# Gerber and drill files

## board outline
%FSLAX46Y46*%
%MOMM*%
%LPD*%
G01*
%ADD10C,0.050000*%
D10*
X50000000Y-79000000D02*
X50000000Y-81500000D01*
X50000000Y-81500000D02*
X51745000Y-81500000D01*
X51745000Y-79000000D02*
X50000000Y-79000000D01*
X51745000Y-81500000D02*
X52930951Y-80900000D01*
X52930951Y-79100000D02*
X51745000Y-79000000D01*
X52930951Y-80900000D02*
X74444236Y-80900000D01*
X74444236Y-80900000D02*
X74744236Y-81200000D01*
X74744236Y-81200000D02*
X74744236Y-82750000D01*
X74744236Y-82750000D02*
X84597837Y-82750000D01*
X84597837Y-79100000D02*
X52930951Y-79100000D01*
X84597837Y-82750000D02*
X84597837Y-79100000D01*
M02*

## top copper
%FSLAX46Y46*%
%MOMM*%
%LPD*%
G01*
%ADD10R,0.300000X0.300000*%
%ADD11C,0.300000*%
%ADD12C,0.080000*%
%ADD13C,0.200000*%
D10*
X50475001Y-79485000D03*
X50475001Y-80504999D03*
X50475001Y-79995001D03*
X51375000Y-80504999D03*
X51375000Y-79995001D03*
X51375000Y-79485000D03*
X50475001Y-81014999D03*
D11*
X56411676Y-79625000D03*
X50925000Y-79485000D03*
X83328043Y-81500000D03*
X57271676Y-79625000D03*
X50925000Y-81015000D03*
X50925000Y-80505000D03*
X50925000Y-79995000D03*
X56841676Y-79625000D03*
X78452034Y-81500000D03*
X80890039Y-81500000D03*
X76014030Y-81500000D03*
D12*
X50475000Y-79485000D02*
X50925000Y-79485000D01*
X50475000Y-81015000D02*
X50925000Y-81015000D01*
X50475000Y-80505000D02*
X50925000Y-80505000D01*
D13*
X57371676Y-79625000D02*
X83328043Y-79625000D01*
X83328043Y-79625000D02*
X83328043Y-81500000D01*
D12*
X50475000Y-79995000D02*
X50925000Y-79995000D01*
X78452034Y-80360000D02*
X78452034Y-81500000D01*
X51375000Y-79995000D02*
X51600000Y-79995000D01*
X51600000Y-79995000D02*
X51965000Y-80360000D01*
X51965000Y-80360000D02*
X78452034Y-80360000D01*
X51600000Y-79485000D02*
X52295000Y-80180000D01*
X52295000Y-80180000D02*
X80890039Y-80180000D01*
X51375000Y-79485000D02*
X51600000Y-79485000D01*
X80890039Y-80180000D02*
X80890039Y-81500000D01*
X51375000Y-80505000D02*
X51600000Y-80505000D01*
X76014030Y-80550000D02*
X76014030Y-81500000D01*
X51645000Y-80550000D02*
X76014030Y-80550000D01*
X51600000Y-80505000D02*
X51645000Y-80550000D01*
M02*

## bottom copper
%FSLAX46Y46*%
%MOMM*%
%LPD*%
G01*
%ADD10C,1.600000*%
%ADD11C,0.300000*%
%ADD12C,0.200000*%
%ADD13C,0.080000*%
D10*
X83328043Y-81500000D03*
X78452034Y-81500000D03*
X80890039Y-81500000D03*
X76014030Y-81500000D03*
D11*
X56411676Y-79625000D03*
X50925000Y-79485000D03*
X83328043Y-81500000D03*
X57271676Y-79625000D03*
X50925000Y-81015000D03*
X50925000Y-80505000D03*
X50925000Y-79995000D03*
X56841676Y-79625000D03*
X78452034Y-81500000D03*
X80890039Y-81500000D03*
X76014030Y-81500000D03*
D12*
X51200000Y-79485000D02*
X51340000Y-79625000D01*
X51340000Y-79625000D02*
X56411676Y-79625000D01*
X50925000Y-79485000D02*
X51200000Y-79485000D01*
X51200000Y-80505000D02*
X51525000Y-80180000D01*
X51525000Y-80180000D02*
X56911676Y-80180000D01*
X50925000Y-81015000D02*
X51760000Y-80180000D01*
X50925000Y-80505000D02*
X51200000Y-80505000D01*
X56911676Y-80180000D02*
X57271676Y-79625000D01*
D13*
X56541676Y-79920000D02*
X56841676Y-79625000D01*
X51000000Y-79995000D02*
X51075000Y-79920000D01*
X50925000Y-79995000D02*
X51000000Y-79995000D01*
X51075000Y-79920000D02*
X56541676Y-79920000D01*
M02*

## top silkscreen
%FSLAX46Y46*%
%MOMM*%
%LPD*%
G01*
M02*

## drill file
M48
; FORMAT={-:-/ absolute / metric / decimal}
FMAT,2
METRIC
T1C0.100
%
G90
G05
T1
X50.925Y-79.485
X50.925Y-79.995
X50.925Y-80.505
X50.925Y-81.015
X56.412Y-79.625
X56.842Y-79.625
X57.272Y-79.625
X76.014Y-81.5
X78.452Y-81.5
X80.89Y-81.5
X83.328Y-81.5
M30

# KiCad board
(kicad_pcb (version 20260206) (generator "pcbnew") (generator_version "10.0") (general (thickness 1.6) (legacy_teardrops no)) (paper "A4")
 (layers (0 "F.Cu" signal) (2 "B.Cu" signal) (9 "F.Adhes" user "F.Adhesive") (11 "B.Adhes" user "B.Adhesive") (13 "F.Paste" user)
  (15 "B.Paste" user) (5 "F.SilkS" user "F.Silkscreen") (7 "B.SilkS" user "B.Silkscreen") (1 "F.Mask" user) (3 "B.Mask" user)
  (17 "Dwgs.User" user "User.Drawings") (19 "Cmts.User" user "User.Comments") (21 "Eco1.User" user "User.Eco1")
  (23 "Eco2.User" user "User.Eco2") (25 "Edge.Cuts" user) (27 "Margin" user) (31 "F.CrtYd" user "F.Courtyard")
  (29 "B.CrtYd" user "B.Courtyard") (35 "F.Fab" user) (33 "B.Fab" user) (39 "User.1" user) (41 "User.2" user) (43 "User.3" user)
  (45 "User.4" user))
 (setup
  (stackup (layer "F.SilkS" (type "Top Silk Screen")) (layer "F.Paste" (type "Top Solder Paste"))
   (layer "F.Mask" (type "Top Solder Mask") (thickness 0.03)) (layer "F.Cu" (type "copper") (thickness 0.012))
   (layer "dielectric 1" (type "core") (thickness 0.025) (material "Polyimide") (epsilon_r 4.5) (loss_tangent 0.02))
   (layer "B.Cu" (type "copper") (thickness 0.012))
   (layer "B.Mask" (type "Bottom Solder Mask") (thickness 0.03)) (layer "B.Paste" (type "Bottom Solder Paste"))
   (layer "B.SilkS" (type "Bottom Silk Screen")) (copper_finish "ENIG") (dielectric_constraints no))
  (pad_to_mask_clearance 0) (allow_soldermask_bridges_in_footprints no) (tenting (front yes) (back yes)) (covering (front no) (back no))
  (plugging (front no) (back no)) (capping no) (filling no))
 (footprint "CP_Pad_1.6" (layer "F.Cu") (at 83.328043 81.5)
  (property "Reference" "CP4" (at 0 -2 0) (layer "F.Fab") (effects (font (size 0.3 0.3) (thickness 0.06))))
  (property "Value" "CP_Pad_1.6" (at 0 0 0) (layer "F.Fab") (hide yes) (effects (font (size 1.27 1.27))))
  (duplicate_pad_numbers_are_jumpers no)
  (pad "1" smd circle (at 0 0) (size 1.6 1.6) (layers "B.Cu" "B.Mask") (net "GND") (solder_mask_margin 0.1)))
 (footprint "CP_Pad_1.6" (layer "F.Cu") (at 78.452034 81.5)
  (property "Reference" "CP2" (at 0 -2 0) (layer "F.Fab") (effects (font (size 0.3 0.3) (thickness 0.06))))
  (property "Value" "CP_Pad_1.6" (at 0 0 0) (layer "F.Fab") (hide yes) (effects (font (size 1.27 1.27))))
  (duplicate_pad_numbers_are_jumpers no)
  (pad "1" smd circle (at 0 0) (size 1.6 1.6) (layers "B.Cu" "B.Mask") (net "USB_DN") (solder_mask_margin 0.1)))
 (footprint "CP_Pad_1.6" (layer "F.Cu") (at 80.890039 81.5)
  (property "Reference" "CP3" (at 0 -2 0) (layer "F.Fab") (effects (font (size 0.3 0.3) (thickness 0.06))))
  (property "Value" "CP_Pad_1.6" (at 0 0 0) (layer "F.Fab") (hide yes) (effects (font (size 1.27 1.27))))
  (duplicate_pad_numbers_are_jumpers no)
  (pad "1" smd circle (at 0 0) (size 1.6 1.6) (layers "B.Cu" "B.Mask") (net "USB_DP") (solder_mask_margin 0.1)))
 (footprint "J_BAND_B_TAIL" (layer "F.Cu") (at 50.9 80.25)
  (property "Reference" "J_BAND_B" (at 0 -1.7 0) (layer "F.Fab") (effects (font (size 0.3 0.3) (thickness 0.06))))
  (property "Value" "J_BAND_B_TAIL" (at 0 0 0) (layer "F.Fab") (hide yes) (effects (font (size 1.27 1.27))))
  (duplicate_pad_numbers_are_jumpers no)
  (pad "1" smd rect (at -0.424999 -0.765) (size 0.3 0.3) (layers "F.Cu" "F.Mask") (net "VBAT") (solder_mask_margin 0.05)
   (thermal_bridge_angle 45))
  (pad "2" smd rect (at -0.424999 0.254999) (size 0.3 0.3) (layers "F.Cu" "F.Mask") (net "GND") (solder_mask_margin 0.05)
   (thermal_bridge_angle 45))
  (pad "3" smd rect (at -0.424999 -0.254999) (size 0.3 0.3) (layers "F.Cu" "F.Mask") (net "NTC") (solder_mask_margin 0.05)
   (thermal_bridge_angle 45))
  (pad "4" smd rect (at 0.475 0.254999) (size 0.3 0.3) (layers "F.Cu" "F.Mask") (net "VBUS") (solder_mask_margin 0.05)
   (thermal_bridge_angle 45))
  (pad "5" smd rect (at 0.475 -0.254999) (size 0.3 0.3) (layers "F.Cu" "F.Mask") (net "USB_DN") (solder_mask_margin 0.05)
   (thermal_bridge_angle 45))
  (pad "6" smd rect (at 0.475 -0.765) (size 0.3 0.3) (layers "F.Cu" "F.Mask") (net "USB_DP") (solder_mask_margin 0.05)
   (thermal_bridge_angle 45))
  (pad "7" smd rect (at -0.424999 0.764999) (size 0.3 0.3) (layers "F.Cu" "F.Mask") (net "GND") (solder_mask_margin 0.05)
   (thermal_bridge_angle 45)))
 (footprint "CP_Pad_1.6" (layer "F.Cu") (at 76.01403 81.5)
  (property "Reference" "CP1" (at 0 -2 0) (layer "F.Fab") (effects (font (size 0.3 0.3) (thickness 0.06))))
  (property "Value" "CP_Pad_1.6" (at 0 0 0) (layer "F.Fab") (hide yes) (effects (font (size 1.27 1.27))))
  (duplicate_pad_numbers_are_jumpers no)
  (pad "1" smd circle (at 0 0) (size 1.6 1.6) (layers "B.Cu" "B.Mask") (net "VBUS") (solder_mask_margin 0.1)))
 (gr_line (start 50 79) (end 50 81.5) (stroke (width 0.05) (type default)) (layer "Edge.Cuts"))
 (gr_line (start 50 81.5) (end 51.745 81.5) (stroke (width 0.05) (type default)) (layer "Edge.Cuts"))
 (gr_line (start 51.745 79) (end 50 79) (stroke (width 0.05) (type default)) (layer "Edge.Cuts"))
 (gr_line (start 51.745 81.5) (end 52.930951 80.9) (stroke (width 0.05) (type default)) (layer "Edge.Cuts"))
 (gr_line (start 52.930951 79.1) (end 51.745 79) (stroke (width 0.05) (type default)) (layer "Edge.Cuts"))
 (gr_line (start 52.930951 80.9) (end 74.444236 80.9) (stroke (width 0.05) (type default)) (layer "Edge.Cuts"))
 (gr_line (start 74.444236 80.9) (end 74.744236 81.2) (stroke (width 0.05) (type default)) (layer "Edge.Cuts"))
 (gr_line (start 74.744236 81.2) (end 74.744236 82.75) (stroke (width 0.05) (type default)) (layer "Edge.Cuts"))
 (gr_line (start 74.744236 82.75) (end 84.597837 82.75) (stroke (width 0.05) (type default)) (layer "Edge.Cuts"))
 (gr_line (start 84.597837 79.1) (end 52.930951 79.1) (stroke (width 0.05) (type default)) (layer "Edge.Cuts"))
 (gr_line (start 84.597837 82.75) (end 84.597837 79.1) (stroke (width 0.05) (type default)) (layer "Edge.Cuts"))
 (segment (start 50.475 79.485) (end 50.925 79.485) (width 0.08) (layer "F.Cu") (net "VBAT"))
 (via (at 56.411676 79.625) (size 0.3) (drill 0.1) (layers "F.Cu" "B.Cu") (tenting (front yes) (back yes)) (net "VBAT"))
 (via (at 50.925 79.485) (size 0.3) (drill 0.1) (layers "F.Cu" "B.Cu") (tenting (front yes) (back yes)) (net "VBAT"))
 (segment (start 51.2 79.485) (end 51.34 79.625) (width 0.2) (layer "B.Cu") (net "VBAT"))
 (segment (start 51.34 79.625) (end 56.411676 79.625) (width 0.2) (layer "B.Cu") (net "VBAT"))
 (segment (start 50.925 79.485) (end 51.2 79.485) (width 0.2) (layer "B.Cu") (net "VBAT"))
 (segment (start 50.475 81.015) (end 50.925 81.015) (width 0.08) (layer "F.Cu") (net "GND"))
 (segment (start 50.475 80.505) (end 50.925 80.505) (width 0.08) (layer "F.Cu") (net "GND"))
 (segment (start 57.371676 79.625) (end 83.328043 79.625) (width 0.2) (layer "F.Cu") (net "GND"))
 (segment (start 83.328043 79.625) (end 83.328043 81.5) (width 0.2) (layer "F.Cu") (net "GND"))
 (via (at 83.328043 81.5) (size 0.3) (drill 0.1) (layers "F.Cu" "B.Cu") (tenting (front yes) (back yes)) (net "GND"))
 (via (at 57.271676 79.625) (size 0.3) (drill 0.1) (layers "F.Cu" "B.Cu") (tenting (front yes) (back yes)) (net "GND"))
 (via (at 50.925 81.015) (size 0.3) (drill 0.1) (layers "F.Cu" "B.Cu") (tenting (front yes) (back yes)) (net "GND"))
 (via (at 50.925 80.505) (size 0.3) (drill 0.1) (layers "F.Cu" "B.Cu") (tenting (front yes) (back yes)) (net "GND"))
 (segment (start 51.2 80.505) (end 51.525 80.18) (width 0.2) (layer "B.Cu") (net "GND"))
 (segment (start 51.525 80.18) (end 56.911676 80.18) (width 0.2) (layer "B.Cu") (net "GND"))
 (segment (start 50.925 81.015) (end 51.76 80.18) (width 0.2) (layer "B.Cu") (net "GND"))
 (segment (start 50.925 80.505) (end 51.2 80.505) (width 0.2) (layer "B.Cu") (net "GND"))
 (segment (start 56.911676 80.18) (end 57.271676 79.625) (width 0.2) (layer "B.Cu") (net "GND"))
 (segment (start 50.475 79.995) (end 50.925 79.995) (width 0.08) (layer "F.Cu") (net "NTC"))
 (via (at 50.925 79.995) (size 0.3) (drill 0.1) (layers "F.Cu" "B.Cu") (tenting (front yes) (back yes)) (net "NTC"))
 (via (at 56.841676 79.625) (size 0.3) (drill 0.1) (layers "F.Cu" "B.Cu") (tenting (front yes) (back yes)) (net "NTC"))
 (segment (start 56.541676 79.92) (end 56.841676 79.625) (width 0.08) (layer "B.Cu") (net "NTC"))
 (segment (start 51 79.995) (end 51.075 79.92) (width 0.08) (layer "B.Cu") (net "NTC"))
 (segment (start 50.925 79.995) (end 51 79.995) (width 0.08) (layer "B.Cu") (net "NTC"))
 (segment (start 51.075 79.92) (end 56.541676 79.92) (width 0.08) (layer "B.Cu") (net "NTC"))
 (segment (start 78.452034 80.36) (end 78.452034 81.5) (width 0.08) (layer "F.Cu") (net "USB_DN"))
 (segment (start 51.375 79.995) (end 51.6 79.995) (width 0.08) (layer "F.Cu") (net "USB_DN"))
 (segment (start 51.6 79.995) (end 51.965 80.36) (width 0.08) (layer "F.Cu") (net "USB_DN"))
 (segment (start 51.965 80.36) (end 78.452034 80.36) (width 0.08) (layer "F.Cu") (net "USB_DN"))
 (via (at 78.452034 81.5) (size 0.3) (drill 0.1) (layers "F.Cu" "B.Cu") (tenting (front yes) (back yes)) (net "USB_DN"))
 (segment (start 51.6 79.485) (end 52.295 80.18) (width 0.08) (layer "F.Cu") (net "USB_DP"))
 (segment (start 52.295 80.18) (end 80.890039 80.18) (width 0.08) (layer "F.Cu") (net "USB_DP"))
 (segment (start 51.375 79.485) (end 51.6 79.485) (width 0.08) (layer "F.Cu") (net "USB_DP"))
 (segment (start 80.890039 80.18) (end 80.890039 81.5) (width 0.08) (layer "F.Cu") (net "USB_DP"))
 (via (at 80.890039 81.5) (size 0.3) (drill 0.1) (layers "F.Cu" "B.Cu") (tenting (front yes) (back yes)) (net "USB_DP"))
 (segment (start 51.375 80.505) (end 51.6 80.505) (width 0.08) (layer "F.Cu") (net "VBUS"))
 (segment (start 76.01403 80.55) (end 76.01403 81.5) (width 0.08) (layer "F.Cu") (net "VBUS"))
 (segment (start 51.645 80.55) (end 76.01403 80.55) (width 0.08) (layer "F.Cu") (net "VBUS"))
 (segment (start 51.6 80.505) (end 51.645 80.55) (width 0.08) (layer "F.Cu") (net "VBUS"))
 (via (at 76.01403 81.5) (size 0.3) (drill 0.1) (layers "F.Cu" "B.Cu") (tenting (front yes) (back yes)) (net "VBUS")))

